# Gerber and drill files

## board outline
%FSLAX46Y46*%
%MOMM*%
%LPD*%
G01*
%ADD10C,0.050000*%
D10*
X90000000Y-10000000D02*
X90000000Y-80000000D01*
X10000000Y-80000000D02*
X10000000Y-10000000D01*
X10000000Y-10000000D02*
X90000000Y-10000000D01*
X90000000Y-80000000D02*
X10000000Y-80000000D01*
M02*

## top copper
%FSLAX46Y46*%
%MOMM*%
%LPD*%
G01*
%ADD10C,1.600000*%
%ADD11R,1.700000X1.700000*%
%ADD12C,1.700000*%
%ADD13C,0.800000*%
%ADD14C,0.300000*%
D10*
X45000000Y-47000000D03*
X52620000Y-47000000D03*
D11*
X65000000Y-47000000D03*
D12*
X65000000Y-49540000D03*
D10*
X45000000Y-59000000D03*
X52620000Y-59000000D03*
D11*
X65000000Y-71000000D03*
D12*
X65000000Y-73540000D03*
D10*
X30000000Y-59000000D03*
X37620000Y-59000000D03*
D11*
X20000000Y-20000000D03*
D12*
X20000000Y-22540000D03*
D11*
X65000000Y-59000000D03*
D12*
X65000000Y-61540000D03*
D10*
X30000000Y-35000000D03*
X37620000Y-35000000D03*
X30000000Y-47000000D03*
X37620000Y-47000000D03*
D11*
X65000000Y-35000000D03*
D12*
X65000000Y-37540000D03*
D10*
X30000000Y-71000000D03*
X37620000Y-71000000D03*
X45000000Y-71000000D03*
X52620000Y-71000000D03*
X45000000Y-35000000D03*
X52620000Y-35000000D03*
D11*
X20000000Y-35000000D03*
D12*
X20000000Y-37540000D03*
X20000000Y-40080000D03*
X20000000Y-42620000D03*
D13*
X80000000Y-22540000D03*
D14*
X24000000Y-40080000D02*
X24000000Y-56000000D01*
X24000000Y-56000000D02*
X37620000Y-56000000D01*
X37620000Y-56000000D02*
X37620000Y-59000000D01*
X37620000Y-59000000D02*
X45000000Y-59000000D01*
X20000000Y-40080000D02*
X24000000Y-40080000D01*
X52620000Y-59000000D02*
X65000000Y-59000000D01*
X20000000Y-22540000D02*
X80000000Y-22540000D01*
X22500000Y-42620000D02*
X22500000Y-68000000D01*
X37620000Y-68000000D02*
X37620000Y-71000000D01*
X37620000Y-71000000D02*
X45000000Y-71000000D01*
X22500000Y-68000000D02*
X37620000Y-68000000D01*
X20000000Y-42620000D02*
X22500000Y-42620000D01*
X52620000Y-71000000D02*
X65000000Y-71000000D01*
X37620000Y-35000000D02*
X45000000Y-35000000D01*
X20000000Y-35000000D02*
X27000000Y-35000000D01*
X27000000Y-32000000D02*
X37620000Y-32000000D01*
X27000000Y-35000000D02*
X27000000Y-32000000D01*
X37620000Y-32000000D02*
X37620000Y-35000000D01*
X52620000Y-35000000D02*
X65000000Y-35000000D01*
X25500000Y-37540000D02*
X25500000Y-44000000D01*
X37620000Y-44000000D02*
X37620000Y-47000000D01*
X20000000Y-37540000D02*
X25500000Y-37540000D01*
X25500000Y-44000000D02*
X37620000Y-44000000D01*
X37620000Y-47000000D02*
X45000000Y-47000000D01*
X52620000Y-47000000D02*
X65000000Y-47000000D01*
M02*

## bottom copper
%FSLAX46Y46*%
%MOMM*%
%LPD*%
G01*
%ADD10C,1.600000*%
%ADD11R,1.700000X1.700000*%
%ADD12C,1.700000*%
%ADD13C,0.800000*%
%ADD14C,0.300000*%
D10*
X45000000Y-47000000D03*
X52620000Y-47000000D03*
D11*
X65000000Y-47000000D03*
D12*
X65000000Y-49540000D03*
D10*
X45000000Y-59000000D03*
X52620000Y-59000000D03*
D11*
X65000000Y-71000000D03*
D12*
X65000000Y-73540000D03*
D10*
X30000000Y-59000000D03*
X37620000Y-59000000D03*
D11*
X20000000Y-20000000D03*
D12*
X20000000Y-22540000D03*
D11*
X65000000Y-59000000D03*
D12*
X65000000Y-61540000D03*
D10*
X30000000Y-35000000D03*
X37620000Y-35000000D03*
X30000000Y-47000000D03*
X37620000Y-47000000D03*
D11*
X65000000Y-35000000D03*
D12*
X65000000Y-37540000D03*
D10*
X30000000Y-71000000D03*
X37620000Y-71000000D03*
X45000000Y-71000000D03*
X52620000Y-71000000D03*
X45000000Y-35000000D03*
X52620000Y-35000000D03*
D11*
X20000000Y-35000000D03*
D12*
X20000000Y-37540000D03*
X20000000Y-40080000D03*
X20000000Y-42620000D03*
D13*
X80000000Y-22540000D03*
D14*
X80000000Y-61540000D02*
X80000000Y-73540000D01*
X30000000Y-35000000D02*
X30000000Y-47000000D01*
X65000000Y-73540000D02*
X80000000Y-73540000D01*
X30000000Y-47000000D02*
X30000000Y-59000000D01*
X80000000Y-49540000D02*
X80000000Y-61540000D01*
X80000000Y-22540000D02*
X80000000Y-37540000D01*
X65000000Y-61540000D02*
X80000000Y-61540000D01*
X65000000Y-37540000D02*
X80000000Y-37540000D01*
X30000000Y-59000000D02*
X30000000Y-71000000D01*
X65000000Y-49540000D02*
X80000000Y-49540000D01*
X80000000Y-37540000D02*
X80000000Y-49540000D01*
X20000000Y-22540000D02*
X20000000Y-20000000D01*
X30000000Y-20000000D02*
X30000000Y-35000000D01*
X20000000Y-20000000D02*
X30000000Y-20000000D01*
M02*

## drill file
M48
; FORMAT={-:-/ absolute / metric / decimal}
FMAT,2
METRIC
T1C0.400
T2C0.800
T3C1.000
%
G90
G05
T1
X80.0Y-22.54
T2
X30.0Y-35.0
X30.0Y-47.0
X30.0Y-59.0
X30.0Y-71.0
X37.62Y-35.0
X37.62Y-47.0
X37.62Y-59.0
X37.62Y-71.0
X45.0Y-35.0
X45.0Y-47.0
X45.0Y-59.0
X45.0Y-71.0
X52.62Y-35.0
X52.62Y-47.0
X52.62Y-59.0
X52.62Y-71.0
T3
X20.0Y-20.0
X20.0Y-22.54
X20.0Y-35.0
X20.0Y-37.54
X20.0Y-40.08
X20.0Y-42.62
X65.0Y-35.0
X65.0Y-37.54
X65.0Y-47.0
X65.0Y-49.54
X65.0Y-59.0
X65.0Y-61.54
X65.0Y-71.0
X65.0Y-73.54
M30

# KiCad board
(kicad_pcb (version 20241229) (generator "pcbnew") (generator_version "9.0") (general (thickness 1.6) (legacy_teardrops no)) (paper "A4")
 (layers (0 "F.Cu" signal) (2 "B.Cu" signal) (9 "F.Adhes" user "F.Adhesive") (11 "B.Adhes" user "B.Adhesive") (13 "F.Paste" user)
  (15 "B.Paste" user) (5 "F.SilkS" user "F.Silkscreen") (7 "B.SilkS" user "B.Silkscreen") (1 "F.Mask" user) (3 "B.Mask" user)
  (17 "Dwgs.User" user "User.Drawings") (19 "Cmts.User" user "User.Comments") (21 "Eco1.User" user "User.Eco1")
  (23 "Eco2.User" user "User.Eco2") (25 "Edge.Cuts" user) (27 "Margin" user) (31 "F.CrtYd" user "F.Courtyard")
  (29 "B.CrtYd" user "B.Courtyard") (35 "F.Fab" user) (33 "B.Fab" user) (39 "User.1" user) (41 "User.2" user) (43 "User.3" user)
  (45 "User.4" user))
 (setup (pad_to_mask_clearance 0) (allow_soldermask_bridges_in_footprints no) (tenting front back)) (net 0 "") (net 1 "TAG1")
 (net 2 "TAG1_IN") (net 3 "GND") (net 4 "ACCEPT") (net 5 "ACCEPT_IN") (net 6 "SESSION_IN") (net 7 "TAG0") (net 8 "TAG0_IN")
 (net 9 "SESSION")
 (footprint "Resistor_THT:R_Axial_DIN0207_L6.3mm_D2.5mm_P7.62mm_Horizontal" (layer "F.Cu") (at 45 47)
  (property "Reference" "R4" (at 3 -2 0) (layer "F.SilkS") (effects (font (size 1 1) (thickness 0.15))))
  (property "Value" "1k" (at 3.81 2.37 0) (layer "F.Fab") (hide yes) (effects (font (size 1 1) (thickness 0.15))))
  (pad "1" thru_hole circle (at 0 0) (size 1.6 1.6) (drill 0.8) (layers "*.Cu" "*.Mask") (remove_unused_layers no) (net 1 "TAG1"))
  (pad "2" thru_hole circle (at 7.62 0) (size 1.6 1.6) (drill 0.8) (layers "*.Cu" "*.Mask") (remove_unused_layers no) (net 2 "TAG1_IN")))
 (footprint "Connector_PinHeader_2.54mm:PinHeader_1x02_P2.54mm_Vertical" (layer "F.Cu") (at 65 47)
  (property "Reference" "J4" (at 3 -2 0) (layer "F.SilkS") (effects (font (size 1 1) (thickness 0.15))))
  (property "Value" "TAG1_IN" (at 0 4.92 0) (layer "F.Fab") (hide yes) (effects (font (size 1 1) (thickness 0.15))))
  (pad "1" thru_hole rect (at 0 0) (size 1.7 1.7) (drill 1) (layers "*.Cu" "*.Mask") (remove_unused_layers no) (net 2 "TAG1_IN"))
  (pad "2" thru_hole circle (at 0 2.54) (size 1.7 1.7) (drill 1) (layers "*.Cu" "*.Mask") (remove_unused_layers no) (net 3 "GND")))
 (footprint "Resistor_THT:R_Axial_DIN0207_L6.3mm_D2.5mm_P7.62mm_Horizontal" (layer "F.Cu") (at 45 59)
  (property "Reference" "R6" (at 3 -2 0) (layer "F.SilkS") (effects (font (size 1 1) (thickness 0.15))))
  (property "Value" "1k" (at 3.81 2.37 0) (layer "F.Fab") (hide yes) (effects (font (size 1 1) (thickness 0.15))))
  (pad "1" thru_hole circle (at 0 0) (size 1.6 1.6) (drill 0.8) (layers "*.Cu" "*.Mask") (remove_unused_layers no) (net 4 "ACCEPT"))
  (pad "2" thru_hole circle (at 7.62 0) (size 1.6 1.6) (drill 0.8) (layers "*.Cu" "*.Mask") (remove_unused_layers no) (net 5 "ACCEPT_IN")))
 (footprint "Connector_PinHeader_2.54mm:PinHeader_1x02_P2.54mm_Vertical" (layer "F.Cu") (at 65 71)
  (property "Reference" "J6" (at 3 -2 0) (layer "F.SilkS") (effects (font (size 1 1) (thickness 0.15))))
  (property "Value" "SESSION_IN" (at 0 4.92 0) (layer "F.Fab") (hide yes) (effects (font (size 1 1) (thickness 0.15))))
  (pad "1" thru_hole rect (at 0 0) (size 1.7 1.7) (drill 1) (layers "*.Cu" "*.Mask") (remove_unused_layers no) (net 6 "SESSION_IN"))
  (pad "2" thru_hole circle (at 0 2.54) (size 1.7 1.7) (drill 1) (layers "*.Cu" "*.Mask") (remove_unused_layers no) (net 3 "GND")))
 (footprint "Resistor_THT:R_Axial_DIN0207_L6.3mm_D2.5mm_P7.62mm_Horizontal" (layer "F.Cu") (at 30 59)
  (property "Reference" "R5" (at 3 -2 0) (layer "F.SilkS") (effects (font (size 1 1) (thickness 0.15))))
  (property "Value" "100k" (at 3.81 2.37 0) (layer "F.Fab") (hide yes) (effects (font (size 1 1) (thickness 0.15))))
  (pad "1" thru_hole circle (at 0 0) (size 1.6 1.6) (drill 0.8) (layers "*.Cu" "*.Mask") (remove_unused_layers no) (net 3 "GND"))
  (pad "2" thru_hole circle (at 7.62 0) (size 1.6 1.6) (drill 0.8) (layers "*.Cu" "*.Mask") (remove_unused_layers no) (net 4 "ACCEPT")))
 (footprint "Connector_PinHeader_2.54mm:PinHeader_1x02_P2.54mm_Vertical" (layer "F.Cu") (at 20 20)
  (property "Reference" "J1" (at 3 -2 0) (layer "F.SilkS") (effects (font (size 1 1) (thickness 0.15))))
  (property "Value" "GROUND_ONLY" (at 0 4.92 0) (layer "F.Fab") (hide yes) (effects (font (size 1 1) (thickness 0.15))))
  (pad "1" thru_hole rect (at 0 0) (size 1.7 1.7) (drill 1) (layers "*.Cu" "*.Mask") (remove_unused_layers no) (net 3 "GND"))
  (pad "2" thru_hole circle (at 0 2.54) (size 1.7 1.7) (drill 1) (layers "*.Cu" "*.Mask") (remove_unused_layers no) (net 3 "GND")))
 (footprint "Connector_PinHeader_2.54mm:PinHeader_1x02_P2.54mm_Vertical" (layer "F.Cu") (at 65 59)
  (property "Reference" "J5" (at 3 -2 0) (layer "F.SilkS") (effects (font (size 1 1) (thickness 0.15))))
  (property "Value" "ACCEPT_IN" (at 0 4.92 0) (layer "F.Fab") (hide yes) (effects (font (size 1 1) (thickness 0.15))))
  (pad "1" thru_hole rect (at 0 0) (size 1.7 1.7) (drill 1) (layers "*.Cu" "*.Mask") (remove_unused_layers no) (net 5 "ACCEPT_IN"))
  (pad "2" thru_hole circle (at 0 2.54) (size 1.7 1.7) (drill 1) (layers "*.Cu" "*.Mask") (remove_unused_layers no) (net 3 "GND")))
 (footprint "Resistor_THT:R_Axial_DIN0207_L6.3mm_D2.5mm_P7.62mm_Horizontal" (layer "F.Cu") (at 30 35)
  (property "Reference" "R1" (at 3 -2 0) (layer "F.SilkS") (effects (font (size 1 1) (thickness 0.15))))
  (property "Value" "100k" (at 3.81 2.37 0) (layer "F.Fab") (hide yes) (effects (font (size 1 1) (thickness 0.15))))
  (pad "1" thru_hole circle (at 0 0) (size 1.6 1.6) (drill 0.8) (layers "*.Cu" "*.Mask") (remove_unused_layers no) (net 3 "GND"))
  (pad "2" thru_hole circle (at 7.62 0) (size 1.6 1.6) (drill 0.8) (layers "*.Cu" "*.Mask") (remove_unused_layers no) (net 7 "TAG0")))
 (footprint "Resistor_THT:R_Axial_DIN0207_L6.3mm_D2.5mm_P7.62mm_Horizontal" (layer "F.Cu") (at 30 47)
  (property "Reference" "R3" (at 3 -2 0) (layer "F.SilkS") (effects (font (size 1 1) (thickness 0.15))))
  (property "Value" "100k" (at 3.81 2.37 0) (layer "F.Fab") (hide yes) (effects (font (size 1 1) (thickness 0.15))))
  (pad "1" thru_hole circle (at 0 0) (size 1.6 1.6) (drill 0.8) (layers "*.Cu" "*.Mask") (remove_unused_layers no) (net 3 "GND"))
  (pad "2" thru_hole circle (at 7.62 0) (size 1.6 1.6) (drill 0.8) (layers "*.Cu" "*.Mask") (remove_unused_layers no) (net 1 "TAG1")))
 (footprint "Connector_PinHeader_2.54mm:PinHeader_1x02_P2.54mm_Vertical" (layer "F.Cu") (at 65 35)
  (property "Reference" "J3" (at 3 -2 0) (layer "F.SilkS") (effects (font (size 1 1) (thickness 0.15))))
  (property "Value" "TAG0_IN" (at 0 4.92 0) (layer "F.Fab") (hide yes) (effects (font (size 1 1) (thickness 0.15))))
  (pad "1" thru_hole rect (at 0 0) (size 1.7 1.7) (drill 1) (layers "*.Cu" "*.Mask") (remove_unused_layers no) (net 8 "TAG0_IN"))
  (pad "2" thru_hole circle (at 0 2.54) (size 1.7 1.7) (drill 1) (layers "*.Cu" "*.Mask") (remove_unused_layers no) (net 3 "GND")))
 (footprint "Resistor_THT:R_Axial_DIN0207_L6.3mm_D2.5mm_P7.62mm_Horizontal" (layer "F.Cu") (at 30 71)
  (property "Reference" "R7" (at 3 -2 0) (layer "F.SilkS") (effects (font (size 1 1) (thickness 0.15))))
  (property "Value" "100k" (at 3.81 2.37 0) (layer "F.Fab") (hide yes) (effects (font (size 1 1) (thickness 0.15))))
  (pad "1" thru_hole circle (at 0 0) (size 1.6 1.6) (drill 0.8) (layers "*.Cu" "*.Mask") (remove_unused_layers no) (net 3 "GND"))
  (pad "2" thru_hole circle (at 7.62 0) (size 1.6 1.6) (drill 0.8) (layers "*.Cu" "*.Mask") (remove_unused_layers no) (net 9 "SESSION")))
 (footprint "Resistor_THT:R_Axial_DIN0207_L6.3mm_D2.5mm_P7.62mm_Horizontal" (layer "F.Cu") (at 45 71)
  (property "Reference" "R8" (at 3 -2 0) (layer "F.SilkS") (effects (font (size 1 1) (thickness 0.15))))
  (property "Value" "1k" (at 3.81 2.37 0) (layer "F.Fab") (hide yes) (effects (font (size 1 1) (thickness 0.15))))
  (pad "1" thru_hole circle (at 0 0) (size 1.6 1.6) (drill 0.8) (layers "*.Cu" "*.Mask") (remove_unused_layers no) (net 9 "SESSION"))
  (pad "2" thru_hole circle (at 7.62 0) (size 1.6 1.6) (drill 0.8) (layers "*.Cu" "*.Mask") (remove_unused_layers no) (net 6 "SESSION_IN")))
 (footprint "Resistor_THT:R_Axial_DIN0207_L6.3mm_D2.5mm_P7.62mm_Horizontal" (layer "F.Cu") (at 45 35)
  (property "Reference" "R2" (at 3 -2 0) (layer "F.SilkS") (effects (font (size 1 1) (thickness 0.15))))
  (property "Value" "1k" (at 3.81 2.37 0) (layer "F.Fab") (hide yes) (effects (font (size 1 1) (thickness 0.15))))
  (pad "1" thru_hole circle (at 0 0) (size 1.6 1.6) (drill 0.8) (layers "*.Cu" "*.Mask") (remove_unused_layers no) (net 7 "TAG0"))
  (pad "2" thru_hole circle (at 7.62 0) (size 1.6 1.6) (drill 0.8) (layers "*.Cu" "*.Mask") (remove_unused_layers no) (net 8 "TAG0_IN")))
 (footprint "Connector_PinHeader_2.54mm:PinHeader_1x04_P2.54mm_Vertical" (layer "F.Cu") (at 20 35)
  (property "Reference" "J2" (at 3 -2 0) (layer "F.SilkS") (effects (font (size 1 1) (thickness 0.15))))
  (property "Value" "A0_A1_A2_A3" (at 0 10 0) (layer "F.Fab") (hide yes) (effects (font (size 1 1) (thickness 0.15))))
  (pad "1" thru_hole rect (at 0 0) (size 1.7 1.7) (drill 1) (layers "*.Cu" "*.Mask") (remove_unused_layers no) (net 7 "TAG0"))
  (pad "2" thru_hole circle (at 0 2.54) (size 1.7 1.7) (drill 1) (layers "*.Cu" "*.Mask") (remove_unused_layers no) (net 1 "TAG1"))
  (pad "3" thru_hole circle (at 0 5.08) (size 1.7 1.7) (drill 1) (layers "*.Cu" "*.Mask") (remove_unused_layers no) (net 4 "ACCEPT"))
  (pad "4" thru_hole circle (at 0 7.62) (size 1.7 1.7) (drill 1) (layers "*.Cu" "*.Mask") (remove_unused_layers no) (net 9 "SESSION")))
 (gr_line (start 90 10) (end 90 80) (stroke (width 0.05) (type default)) (layer "Edge.Cuts"))
 (gr_line (start 10 80) (end 10 10) (stroke (width 0.05) (type default)) (layer "Edge.Cuts"))
 (gr_line (start 10 10) (end 90 10) (stroke (width 0.05) (type default)) (layer "Edge.Cuts"))
 (gr_line (start 90 80) (end 10 80) (stroke (width 0.05) (type default)) (layer "Edge.Cuts"))
 (segment (start 24 40.08) (end 24 56) (width 0.3) (layer "F.Cu") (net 4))
 (segment (start 24 56) (end 37.62 56) (width 0.3) (layer "F.Cu") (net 4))
 (segment (start 37.62 56) (end 37.62 59) (width 0.3) (layer "F.Cu") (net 4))
 (segment (start 37.62 59) (end 45 59) (width 0.3) (layer "F.Cu") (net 4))
 (segment (start 20 40.08) (end 24 40.08) (width 0.3) (layer "F.Cu") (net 4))
 (segment (start 52.62 59) (end 65 59) (width 0.3) (layer "F.Cu") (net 5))
 (segment (start 20 22.54) (end 80 22.54) (width 0.3) (layer "F.Cu") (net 3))
 (via (at 80 22.54) (size 0.8) (drill 0.4) (layers "F.Cu" "B.Cu") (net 3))
 (segment (start 80 61.54) (end 80 73.54) (width 0.3) (layer "B.Cu") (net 3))
 (segment (start 30 35) (end 30 47) (width 0.3) (layer "B.Cu") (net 3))
 (segment (start 65 73.54) (end 80 73.54) (width 0.3) (layer "B.Cu") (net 3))
 (segment (start 30 47) (end 30 59) (width 0.3) (layer "B.Cu") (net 3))
 (segment (start 80 49.54) (end 80 61.54) (width 0.3) (layer "B.Cu") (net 3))
 (segment (start 80 22.54) (end 80 37.54) (width 0.3) (layer "B.Cu") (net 3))
 (segment (start 65 61.54) (end 80 61.54) (width 0.3) (layer "B.Cu") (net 3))
 (segment (start 65 37.54) (end 80 37.54) (width 0.3) (layer "B.Cu") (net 3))
 (segment (start 30 59) (end 30 71) (width 0.3) (layer "B.Cu") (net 3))
 (segment (start 65 49.54) (end 80 49.54) (width 0.3) (layer "B.Cu") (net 3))
 (segment (start 80 37.54) (end 80 49.54) (width 0.3) (layer "B.Cu") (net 3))
 (segment (start 20 22.54) (end 20 20) (width 0.3) (layer "B.Cu") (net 3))
 (segment (start 30 20) (end 30 35) (width 0.3) (layer "B.Cu") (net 3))
 (segment (start 20 20) (end 30 20) (width 0.3) (layer "B.Cu") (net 3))
 (segment (start 22.5 42.62) (end 22.5 68) (width 0.3) (layer "F.Cu") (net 9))
 (segment (start 37.62 68) (end 37.62 71) (width 0.3) (layer "F.Cu") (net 9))
 (segment (start 37.62 71) (end 45 71) (width 0.3) (layer "F.Cu") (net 9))
 (segment (start 22.5 68) (end 37.62 68) (width 0.3) (layer "F.Cu") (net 9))
 (segment (start 20 42.62) (end 22.5 42.62) (width 0.3) (layer "F.Cu") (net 9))
 (segment (start 52.62 71) (end 65 71) (width 0.3) (layer "F.Cu") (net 6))
 (segment (start 37.62 35) (end 45 35) (width 0.3) (layer "F.Cu") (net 7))
 (segment (start 20 35) (end 27 35) (width 0.3) (layer "F.Cu") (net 7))
 (segment (start 27 32) (end 37.62 32) (width 0.3) (layer "F.Cu") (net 7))
 (segment (start 27 35) (end 27 32) (width 0.3) (layer "F.Cu") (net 7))
 (segment (start 37.62 32) (end 37.62 35) (width 0.3) (layer "F.Cu") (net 7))
 (segment (start 52.62 35) (end 65 35) (width 0.3) (layer "F.Cu") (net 8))
 (segment (start 25.5 37.54) (end 25.5 44) (width 0.3) (layer "F.Cu") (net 1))
 (segment (start 37.62 44) (end 37.62 47) (width 0.3) (layer "F.Cu") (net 1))
 (segment (start 20 37.54) (end 25.5 37.54) (width 0.3) (layer "F.Cu") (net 1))
 (segment (start 25.5 44) (end 37.62 44) (width 0.3) (layer "F.Cu") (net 1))
 (segment (start 37.62 47) (end 45 47) (width 0.3) (layer "F.Cu") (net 1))
 (segment (start 52.62 47) (end 65 47) (width 0.3) (layer "F.Cu") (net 2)))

